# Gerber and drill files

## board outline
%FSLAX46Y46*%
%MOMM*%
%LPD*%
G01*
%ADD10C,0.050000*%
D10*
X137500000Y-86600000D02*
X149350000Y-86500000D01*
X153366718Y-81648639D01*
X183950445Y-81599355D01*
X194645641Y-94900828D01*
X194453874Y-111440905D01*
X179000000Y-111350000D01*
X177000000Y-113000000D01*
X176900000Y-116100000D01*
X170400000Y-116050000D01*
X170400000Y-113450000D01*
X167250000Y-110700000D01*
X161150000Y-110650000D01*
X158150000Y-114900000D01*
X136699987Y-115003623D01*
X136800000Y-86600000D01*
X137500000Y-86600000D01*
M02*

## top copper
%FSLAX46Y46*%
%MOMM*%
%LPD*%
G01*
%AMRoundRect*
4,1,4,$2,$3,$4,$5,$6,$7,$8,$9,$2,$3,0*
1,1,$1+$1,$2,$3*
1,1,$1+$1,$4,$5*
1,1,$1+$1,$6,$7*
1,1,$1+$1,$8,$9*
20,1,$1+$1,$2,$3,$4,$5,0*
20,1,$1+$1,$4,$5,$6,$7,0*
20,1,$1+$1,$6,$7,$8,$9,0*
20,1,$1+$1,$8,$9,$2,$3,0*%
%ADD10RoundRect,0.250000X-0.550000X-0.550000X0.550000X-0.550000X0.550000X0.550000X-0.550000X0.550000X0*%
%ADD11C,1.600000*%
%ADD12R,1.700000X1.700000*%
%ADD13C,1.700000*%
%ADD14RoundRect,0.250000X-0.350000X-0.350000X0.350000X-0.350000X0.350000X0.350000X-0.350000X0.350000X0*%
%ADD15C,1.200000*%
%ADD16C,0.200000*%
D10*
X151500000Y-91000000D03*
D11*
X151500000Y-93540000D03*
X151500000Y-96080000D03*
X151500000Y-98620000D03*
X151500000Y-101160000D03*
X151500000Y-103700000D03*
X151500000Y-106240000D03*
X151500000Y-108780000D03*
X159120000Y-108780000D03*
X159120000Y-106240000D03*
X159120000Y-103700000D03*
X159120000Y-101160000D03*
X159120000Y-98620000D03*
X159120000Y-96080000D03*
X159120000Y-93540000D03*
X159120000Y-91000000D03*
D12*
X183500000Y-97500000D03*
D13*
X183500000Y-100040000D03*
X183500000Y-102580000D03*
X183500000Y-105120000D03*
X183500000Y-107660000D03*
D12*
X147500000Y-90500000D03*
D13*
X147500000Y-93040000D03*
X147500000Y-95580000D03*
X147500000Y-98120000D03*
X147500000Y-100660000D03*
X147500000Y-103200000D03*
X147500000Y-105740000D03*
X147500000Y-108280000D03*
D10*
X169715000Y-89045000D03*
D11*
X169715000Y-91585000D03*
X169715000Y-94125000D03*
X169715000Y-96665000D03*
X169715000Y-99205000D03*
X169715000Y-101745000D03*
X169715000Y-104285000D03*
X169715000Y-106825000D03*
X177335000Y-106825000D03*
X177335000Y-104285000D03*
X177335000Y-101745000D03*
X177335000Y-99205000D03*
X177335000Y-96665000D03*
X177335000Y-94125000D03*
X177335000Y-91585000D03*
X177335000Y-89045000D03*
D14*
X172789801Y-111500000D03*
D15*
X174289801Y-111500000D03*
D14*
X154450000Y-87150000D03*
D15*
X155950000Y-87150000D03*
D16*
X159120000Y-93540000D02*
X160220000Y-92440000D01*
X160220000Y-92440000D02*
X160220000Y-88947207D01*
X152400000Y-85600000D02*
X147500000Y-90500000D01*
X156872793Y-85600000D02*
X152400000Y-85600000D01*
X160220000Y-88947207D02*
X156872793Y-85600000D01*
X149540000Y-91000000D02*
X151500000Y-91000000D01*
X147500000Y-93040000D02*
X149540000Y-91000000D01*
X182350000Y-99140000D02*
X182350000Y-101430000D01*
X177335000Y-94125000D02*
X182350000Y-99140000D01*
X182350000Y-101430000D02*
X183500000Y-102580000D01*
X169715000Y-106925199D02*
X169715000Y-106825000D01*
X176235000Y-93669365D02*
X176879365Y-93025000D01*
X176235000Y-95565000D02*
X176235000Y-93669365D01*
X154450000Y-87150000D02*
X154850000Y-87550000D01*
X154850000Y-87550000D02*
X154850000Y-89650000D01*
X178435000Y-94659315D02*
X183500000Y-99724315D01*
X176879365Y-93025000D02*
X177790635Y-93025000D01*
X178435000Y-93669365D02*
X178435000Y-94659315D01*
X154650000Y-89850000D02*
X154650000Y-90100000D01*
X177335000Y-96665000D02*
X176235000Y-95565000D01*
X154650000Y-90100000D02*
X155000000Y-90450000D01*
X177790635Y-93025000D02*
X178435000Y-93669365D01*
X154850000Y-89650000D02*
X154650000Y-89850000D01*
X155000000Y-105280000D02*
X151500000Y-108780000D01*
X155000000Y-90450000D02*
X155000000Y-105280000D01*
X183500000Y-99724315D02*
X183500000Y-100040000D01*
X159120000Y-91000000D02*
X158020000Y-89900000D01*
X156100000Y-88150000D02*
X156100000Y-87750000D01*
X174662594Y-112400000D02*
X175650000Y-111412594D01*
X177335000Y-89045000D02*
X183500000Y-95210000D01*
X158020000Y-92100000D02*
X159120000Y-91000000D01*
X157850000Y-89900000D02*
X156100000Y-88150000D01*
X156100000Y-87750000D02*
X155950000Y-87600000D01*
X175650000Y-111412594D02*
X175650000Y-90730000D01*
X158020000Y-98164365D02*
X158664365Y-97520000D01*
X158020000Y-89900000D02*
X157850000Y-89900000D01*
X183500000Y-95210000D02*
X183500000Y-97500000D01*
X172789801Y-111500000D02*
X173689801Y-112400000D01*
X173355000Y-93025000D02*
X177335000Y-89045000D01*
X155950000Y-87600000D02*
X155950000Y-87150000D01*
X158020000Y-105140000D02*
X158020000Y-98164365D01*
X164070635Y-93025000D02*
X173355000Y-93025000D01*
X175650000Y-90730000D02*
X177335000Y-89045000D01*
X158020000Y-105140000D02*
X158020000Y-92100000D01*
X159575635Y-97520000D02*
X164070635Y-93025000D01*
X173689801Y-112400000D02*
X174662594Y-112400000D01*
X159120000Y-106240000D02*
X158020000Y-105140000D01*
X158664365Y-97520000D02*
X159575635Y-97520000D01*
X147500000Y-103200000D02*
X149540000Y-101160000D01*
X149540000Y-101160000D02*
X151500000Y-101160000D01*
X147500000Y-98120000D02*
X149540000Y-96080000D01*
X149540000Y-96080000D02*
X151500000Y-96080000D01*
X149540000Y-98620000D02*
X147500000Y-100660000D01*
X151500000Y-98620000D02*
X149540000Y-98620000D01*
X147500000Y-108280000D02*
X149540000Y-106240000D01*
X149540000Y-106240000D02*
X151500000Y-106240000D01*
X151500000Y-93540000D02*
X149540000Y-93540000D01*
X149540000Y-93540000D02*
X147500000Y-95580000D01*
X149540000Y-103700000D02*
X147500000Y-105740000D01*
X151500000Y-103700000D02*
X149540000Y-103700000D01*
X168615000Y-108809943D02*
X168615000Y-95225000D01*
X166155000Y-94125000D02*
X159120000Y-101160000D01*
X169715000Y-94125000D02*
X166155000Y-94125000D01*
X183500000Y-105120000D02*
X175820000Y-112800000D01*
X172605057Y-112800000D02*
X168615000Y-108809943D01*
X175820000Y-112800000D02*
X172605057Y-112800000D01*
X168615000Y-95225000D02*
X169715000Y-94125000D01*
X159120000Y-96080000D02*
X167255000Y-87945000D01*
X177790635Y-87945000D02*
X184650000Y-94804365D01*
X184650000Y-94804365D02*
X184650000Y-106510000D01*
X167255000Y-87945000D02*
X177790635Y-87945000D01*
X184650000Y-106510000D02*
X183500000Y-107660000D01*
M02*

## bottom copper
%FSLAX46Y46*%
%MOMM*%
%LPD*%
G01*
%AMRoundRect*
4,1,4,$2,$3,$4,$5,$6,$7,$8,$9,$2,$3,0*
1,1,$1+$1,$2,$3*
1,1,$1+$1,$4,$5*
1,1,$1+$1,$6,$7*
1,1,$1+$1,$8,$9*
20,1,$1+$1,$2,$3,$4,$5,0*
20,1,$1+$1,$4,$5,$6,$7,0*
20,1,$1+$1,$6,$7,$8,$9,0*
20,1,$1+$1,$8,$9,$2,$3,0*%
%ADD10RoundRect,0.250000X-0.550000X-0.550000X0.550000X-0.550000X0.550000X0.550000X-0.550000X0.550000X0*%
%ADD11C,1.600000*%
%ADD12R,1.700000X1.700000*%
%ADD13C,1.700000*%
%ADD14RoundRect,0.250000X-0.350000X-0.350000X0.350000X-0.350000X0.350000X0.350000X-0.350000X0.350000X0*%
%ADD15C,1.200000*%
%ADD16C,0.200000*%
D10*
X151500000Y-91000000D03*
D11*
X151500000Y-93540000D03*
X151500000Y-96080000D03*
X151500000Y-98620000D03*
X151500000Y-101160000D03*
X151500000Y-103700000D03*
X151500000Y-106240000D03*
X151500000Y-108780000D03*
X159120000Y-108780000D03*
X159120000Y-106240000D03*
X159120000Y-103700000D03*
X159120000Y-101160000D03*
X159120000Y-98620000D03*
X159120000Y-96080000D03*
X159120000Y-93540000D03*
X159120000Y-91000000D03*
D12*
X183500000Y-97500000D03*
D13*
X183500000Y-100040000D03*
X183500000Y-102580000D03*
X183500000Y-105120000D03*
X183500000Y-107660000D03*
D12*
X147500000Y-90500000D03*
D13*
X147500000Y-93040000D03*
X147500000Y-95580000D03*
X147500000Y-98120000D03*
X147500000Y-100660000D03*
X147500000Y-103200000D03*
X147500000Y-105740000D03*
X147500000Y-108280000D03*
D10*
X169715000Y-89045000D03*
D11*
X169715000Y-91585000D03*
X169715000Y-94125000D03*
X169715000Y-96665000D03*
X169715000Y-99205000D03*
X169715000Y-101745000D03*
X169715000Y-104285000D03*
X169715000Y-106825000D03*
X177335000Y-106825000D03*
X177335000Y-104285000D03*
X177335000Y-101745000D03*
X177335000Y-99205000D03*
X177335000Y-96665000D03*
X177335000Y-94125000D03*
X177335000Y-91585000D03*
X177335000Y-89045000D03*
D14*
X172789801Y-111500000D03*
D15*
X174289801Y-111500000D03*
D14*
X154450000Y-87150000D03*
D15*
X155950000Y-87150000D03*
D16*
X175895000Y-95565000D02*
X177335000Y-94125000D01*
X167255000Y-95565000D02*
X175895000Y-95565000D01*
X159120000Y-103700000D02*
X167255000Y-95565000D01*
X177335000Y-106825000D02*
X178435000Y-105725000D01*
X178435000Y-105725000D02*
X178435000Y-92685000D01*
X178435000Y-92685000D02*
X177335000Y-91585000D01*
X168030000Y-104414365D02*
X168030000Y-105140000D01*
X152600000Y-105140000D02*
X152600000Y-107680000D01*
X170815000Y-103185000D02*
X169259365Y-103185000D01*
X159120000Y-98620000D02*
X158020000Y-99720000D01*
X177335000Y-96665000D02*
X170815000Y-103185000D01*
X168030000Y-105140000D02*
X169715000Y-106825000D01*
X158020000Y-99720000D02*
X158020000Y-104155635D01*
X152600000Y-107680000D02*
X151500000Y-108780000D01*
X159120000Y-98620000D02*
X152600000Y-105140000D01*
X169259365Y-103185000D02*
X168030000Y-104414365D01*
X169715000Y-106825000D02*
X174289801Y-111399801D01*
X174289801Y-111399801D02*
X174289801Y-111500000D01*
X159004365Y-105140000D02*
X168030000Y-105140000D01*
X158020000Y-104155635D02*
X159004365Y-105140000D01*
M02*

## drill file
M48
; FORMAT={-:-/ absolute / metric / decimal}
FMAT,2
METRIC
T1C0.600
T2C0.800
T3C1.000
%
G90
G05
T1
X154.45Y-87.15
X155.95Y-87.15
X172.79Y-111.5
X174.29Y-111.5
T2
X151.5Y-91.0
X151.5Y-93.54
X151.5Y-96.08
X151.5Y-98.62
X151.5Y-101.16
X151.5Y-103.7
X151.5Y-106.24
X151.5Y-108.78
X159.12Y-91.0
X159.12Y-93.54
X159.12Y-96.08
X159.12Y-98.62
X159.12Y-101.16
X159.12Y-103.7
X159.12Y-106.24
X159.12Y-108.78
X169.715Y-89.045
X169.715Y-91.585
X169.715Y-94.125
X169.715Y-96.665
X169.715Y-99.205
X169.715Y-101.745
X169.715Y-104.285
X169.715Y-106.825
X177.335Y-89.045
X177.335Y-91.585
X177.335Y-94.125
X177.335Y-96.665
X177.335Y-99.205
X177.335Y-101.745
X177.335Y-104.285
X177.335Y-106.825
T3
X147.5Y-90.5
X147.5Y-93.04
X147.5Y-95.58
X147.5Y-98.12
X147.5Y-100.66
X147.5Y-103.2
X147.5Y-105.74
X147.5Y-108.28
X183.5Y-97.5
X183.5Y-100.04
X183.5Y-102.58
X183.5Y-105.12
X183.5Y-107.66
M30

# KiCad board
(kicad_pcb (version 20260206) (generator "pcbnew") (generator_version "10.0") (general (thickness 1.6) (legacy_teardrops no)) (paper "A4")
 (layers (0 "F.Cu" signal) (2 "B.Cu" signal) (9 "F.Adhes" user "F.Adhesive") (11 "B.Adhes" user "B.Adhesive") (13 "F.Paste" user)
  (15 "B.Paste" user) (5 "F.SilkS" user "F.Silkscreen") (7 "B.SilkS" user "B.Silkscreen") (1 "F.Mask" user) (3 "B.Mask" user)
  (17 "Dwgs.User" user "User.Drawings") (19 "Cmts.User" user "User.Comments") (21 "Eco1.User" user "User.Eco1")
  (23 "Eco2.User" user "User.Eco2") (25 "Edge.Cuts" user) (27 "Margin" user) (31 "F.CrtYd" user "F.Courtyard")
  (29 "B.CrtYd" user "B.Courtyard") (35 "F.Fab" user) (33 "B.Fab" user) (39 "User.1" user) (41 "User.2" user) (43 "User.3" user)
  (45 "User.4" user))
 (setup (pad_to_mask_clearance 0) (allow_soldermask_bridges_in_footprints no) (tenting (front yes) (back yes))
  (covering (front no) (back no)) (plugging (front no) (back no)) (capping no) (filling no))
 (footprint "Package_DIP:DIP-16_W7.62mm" (layer "F.Cu") (at 151.5 91)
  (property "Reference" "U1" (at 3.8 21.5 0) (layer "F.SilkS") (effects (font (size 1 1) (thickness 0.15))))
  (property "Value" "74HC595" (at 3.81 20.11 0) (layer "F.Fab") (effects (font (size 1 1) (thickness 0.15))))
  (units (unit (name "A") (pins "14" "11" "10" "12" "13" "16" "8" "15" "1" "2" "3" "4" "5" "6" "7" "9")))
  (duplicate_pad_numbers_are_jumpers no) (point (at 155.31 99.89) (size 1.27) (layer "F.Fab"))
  (pad "1" thru_hole roundrect (at 0 0) (size 1.6 1.6) (drill 0.8) (layers "*.Cu" "*.Mask") (remove_unused_layers no)
   (roundrect_rratio 0.15625) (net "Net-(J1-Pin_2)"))
  (pad "2" thru_hole circle (at 0 2.54) (size 1.6 1.6) (drill 0.8) (layers "*.Cu" "*.Mask") (remove_unused_layers no) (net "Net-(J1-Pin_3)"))
  (pad "3" thru_hole circle (at 0 5.08) (size 1.6 1.6) (drill 0.8) (layers "*.Cu" "*.Mask") (remove_unused_layers no) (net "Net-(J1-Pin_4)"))
  (pad "4" thru_hole circle (at 0 7.62) (size 1.6 1.6) (drill 0.8) (layers "*.Cu" "*.Mask") (remove_unused_layers no) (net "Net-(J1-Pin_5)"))
  (pad "5" thru_hole circle (at 0 10.16) (size 1.6 1.6) (drill 0.8) (layers "*.Cu" "*.Mask") (remove_unused_layers no)
   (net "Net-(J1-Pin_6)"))
  (pad "6" thru_hole circle (at 0 12.7) (size 1.6 1.6) (drill 0.8) (layers "*.Cu" "*.Mask") (remove_unused_layers no) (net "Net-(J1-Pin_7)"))
  (pad "7" thru_hole circle (at 0 15.24) (size 1.6 1.6) (drill 0.8) (layers "*.Cu" "*.Mask") (remove_unused_layers no)
   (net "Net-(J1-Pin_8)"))
  (pad "8" thru_hole circle (at 0 17.78) (size 1.6 1.6) (drill 0.8) (layers "*.Cu" "*.Mask") (remove_unused_layers no) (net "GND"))
  (pad "9" thru_hole circle (at 7.62 17.78) (size 1.6 1.6) (drill 0.8) (layers "*.Cu" "*.Mask") (remove_unused_layers no)
   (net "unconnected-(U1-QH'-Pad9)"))
  (pad "10" thru_hole circle (at 7.62 15.24) (size 1.6 1.6) (drill 0.8) (layers "*.Cu" "*.Mask") (remove_unused_layers no) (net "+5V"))
  (pad "11" thru_hole circle (at 7.62 12.7) (size 1.6 1.6) (drill 0.8) (layers "*.Cu" "*.Mask") (remove_unused_layers no) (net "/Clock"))
  (pad "12" thru_hole circle (at 7.62 10.16) (size 1.6 1.6) (drill 0.8) (layers "*.Cu" "*.Mask") (remove_unused_layers no)
   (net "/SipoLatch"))
  (pad "13" thru_hole circle (at 7.62 7.62) (size 1.6 1.6) (drill 0.8) (layers "*.Cu" "*.Mask") (remove_unused_layers no) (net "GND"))
  (pad "14" thru_hole circle (at 7.62 5.08) (size 1.6 1.6) (drill 0.8) (layers "*.Cu" "*.Mask") (remove_unused_layers no) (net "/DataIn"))
  (pad "15" thru_hole circle (at 7.62 2.54) (size 1.6 1.6) (drill 0.8) (layers "*.Cu" "*.Mask") (remove_unused_layers no)
   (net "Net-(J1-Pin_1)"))
  (pad "16" thru_hole circle (at 7.62 0) (size 1.6 1.6) (drill 0.8) (layers "*.Cu" "*.Mask") (remove_unused_layers no) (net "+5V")))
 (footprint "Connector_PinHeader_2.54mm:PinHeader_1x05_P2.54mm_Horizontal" (layer "F.Cu") (at 183.5 97.5)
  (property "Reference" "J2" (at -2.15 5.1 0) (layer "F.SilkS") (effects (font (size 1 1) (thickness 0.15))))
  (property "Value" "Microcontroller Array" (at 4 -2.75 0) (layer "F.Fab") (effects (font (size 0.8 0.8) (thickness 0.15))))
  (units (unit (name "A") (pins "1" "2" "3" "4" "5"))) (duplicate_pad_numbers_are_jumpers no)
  (pad "1" thru_hole rect (at 0 0) (size 1.7 1.7) (drill 1) (layers "*.Cu" "*.Mask") (remove_unused_layers no) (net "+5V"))
  (pad "2" thru_hole circle (at 0 2.54) (size 1.7 1.7) (drill 1) (layers "*.Cu" "*.Mask") (remove_unused_layers no) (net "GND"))
  (pad "3" thru_hole circle (at 0 5.08) (size 1.7 1.7) (drill 1) (layers "*.Cu" "*.Mask") (remove_unused_layers no) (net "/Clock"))
  (pad "4" thru_hole circle (at 0 7.62) (size 1.7 1.7) (drill 1) (layers "*.Cu" "*.Mask") (remove_unused_layers no) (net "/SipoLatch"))
  (pad "5" thru_hole circle (at 0 10.16) (size 1.7 1.7) (drill 1) (layers "*.Cu" "*.Mask") (remove_unused_layers no) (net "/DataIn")))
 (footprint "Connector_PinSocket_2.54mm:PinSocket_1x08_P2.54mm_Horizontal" (layer "F.Cu") (at 147.5 90.5)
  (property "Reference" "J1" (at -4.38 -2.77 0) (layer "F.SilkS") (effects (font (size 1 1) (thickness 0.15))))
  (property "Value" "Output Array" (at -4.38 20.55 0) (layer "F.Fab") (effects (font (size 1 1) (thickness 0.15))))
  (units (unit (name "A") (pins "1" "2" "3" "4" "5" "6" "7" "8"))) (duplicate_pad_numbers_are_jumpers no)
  (pad "1" thru_hole rect (at 0 0) (size 1.7 1.7) (drill 1) (layers "*.Cu" "*.Mask") (remove_unused_layers no) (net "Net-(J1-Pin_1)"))
  (pad "2" thru_hole circle (at 0 2.54) (size 1.7 1.7) (drill 1) (layers "*.Cu" "*.Mask") (remove_unused_layers no) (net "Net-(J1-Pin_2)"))
  (pad "3" thru_hole circle (at 0 5.08) (size 1.7 1.7) (drill 1) (layers "*.Cu" "*.Mask") (remove_unused_layers no) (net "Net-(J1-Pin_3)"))
  (pad "4" thru_hole circle (at 0 7.62) (size 1.7 1.7) (drill 1) (layers "*.Cu" "*.Mask") (remove_unused_layers no) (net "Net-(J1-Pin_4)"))
  (pad "5" thru_hole circle (at 0 10.16) (size 1.7 1.7) (drill 1) (layers "*.Cu" "*.Mask") (remove_unused_layers no) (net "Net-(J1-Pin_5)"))
  (pad "6" thru_hole circle (at 0 12.7) (size 1.7 1.7) (drill 1) (layers "*.Cu" "*.Mask") (remove_unused_layers no) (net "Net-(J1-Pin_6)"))
  (pad "7" thru_hole circle (at 0 15.24) (size 1.7 1.7) (drill 1) (layers "*.Cu" "*.Mask") (remove_unused_layers no) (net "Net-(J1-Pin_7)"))
  (pad "8" thru_hole circle (at 0 17.78) (size 1.7 1.7) (drill 1) (layers "*.Cu" "*.Mask") (remove_unused_layers no) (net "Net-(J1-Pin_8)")))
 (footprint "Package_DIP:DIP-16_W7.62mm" (layer "F.Cu") (at 169.715 89.045)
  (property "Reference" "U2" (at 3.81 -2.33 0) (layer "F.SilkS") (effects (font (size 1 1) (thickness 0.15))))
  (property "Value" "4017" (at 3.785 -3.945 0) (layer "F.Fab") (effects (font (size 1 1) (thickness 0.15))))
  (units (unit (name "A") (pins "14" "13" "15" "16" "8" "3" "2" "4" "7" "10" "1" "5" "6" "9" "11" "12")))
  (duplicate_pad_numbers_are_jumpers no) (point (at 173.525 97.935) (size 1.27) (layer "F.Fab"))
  (pad "1" thru_hole roundrect (at 0 0) (size 1.6 1.6) (drill 0.8) (layers "*.Cu" "*.Mask") (remove_unused_layers no)
   (roundrect_rratio 0.15625) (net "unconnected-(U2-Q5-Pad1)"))
  (pad "2" thru_hole circle (at 0 2.54) (size 1.6 1.6) (drill 0.8) (layers "*.Cu" "*.Mask") (remove_unused_layers no)
   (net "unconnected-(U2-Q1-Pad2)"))
  (pad "3" thru_hole circle (at 0 5.08) (size 1.6 1.6) (drill 0.8) (layers "*.Cu" "*.Mask") (remove_unused_layers no) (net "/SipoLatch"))
  (pad "4" thru_hole circle (at 0 7.62) (size 1.6 1.6) (drill 0.8) (layers "*.Cu" "*.Mask") (remove_unused_layers no)
   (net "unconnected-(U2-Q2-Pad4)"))
  (pad "5" thru_hole circle (at 0 10.16) (size 1.6 1.6) (drill 0.8) (layers "*.Cu" "*.Mask") (remove_unused_layers no)
   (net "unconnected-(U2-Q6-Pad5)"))
  (pad "6" thru_hole circle (at 0 12.7) (size 1.6 1.6) (drill 0.8) (layers "*.Cu" "*.Mask") (remove_unused_layers no)
   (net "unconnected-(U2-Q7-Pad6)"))
  (pad "7" thru_hole circle (at 0 15.24) (size 1.6 1.6) (drill 0.8) (layers "*.Cu" "*.Mask") (remove_unused_layers no)
   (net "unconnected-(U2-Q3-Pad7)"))
  (pad "8" thru_hole circle (at 0 17.78) (size 1.6 1.6) (drill 0.8) (layers "*.Cu" "*.Mask") (remove_unused_layers no) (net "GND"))
  (pad "9" thru_hole circle (at 7.62 17.78) (size 1.6 1.6) (drill 0.8) (layers "*.Cu" "*.Mask") (remove_unused_layers no)
   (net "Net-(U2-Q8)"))
  (pad "10" thru_hole circle (at 7.62 15.24) (size 1.6 1.6) (drill 0.8) (layers "*.Cu" "*.Mask") (remove_unused_layers no)
   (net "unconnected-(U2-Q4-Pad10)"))
  (pad "11" thru_hole circle (at 7.62 12.7) (size 1.6 1.6) (drill 0.8) (layers "*.Cu" "*.Mask") (remove_unused_layers no)
   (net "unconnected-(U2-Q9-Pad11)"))
  (pad "12" thru_hole circle (at 7.62 10.16) (size 1.6 1.6) (drill 0.8) (layers "*.Cu" "*.Mask") (remove_unused_layers no)
   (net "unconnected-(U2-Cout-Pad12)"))
  (pad "13" thru_hole circle (at 7.62 7.62) (size 1.6 1.6) (drill 0.8) (layers "*.Cu" "*.Mask") (remove_unused_layers no) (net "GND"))
  (pad "14" thru_hole circle (at 7.62 5.08) (size 1.6 1.6) (drill 0.8) (layers "*.Cu" "*.Mask") (remove_unused_layers no) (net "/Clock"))
  (pad "15" thru_hole circle (at 7.62 2.54) (size 1.6 1.6) (drill 0.8) (layers "*.Cu" "*.Mask") (remove_unused_layers no)
   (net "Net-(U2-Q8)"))
  (pad "16" thru_hole circle (at 7.62 0) (size 1.6 1.6) (drill 0.8) (layers "*.Cu" "*.Mask") (remove_unused_layers no) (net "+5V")))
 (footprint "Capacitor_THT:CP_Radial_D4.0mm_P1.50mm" (layer "F.Cu") (at 172.789801 111.5)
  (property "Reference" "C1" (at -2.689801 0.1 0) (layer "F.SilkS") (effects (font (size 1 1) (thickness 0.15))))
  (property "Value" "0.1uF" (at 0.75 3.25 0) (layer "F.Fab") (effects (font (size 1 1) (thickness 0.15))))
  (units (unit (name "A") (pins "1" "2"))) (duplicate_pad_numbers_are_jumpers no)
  (pad "1" thru_hole roundrect (at 0 0) (size 1.2 1.2) (drill 0.6) (layers "*.Cu" "*.Mask") (remove_unused_layers no)
   (roundrect_rratio 0.208333) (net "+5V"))
  (pad "2" thru_hole circle (at 1.5 0) (size 1.2 1.2) (drill 0.6) (layers "*.Cu" "*.Mask") (remove_unused_layers no) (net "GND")))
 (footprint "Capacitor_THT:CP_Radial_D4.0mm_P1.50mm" (layer "F.Cu") (at 154.45 87.15)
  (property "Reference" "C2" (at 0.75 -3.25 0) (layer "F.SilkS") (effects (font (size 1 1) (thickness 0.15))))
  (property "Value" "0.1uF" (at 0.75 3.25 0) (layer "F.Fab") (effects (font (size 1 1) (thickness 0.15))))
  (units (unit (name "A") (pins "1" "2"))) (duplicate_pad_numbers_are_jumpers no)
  (pad "1" thru_hole roundrect (at 0 0) (size 1.2 1.2) (drill 0.6) (layers "*.Cu" "*.Mask") (remove_unused_layers no)
   (roundrect_rratio 0.208333) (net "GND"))
  (pad "2" thru_hole circle (at 1.5 0) (size 1.2 1.2) (drill 0.6) (layers "*.Cu" "*.Mask") (remove_unused_layers no) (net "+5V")))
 (gr_poly
  (pts (xy 137.5 86.6) (xy 149.35 86.5) (xy 153.366718 81.648639) (xy 183.950445 81.599355) (xy 194.645641 94.900828)
   (xy 194.453874 111.440905) (xy 179 111.35) (xy 177 113) (xy 176.9 116.1) (xy 170.4 116.05) (xy 170.4 113.45) (xy 167.25 110.7)
   (xy 161.15 110.65) (xy 158.15 114.9) (xy 136.699987 115.003623) (xy 136.8 86.6))
  (stroke (width 0.05) (type solid)) (fill no) (layer "Edge.Cuts"))
 (segment (start 159.12 93.54) (end 160.22 92.44) (width 0.2) (layer "F.Cu") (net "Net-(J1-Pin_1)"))
 (segment (start 160.22 92.44) (end 160.22 88.947207) (width 0.2) (layer "F.Cu") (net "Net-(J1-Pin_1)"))
 (segment (start 152.4 85.6) (end 147.5 90.5) (width 0.2) (layer "F.Cu") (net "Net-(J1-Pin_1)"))
 (segment (start 156.872793 85.6) (end 152.4 85.6) (width 0.2) (layer "F.Cu") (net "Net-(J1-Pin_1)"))
 (segment (start 160.22 88.947207) (end 156.872793 85.6) (width 0.2) (layer "F.Cu") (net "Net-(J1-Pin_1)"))
 (segment (start 149.54 91) (end 151.5 91) (width 0.2) (layer "F.Cu") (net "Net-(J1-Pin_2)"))
 (segment (start 147.5 93.04) (end 149.54 91) (width 0.2) (layer "F.Cu") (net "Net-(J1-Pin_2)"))
 (segment (start 182.35 99.14) (end 182.35 101.43) (width 0.2) (layer "F.Cu") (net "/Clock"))
 (segment (start 177.335 94.125) (end 182.35 99.14) (width 0.2) (layer "F.Cu") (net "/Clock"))
 (segment (start 182.35 101.43) (end 183.5 102.58) (width 0.2) (layer "F.Cu") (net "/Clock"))
 (segment (start 175.895 95.565) (end 177.335 94.125) (width 0.2) (layer "B.Cu") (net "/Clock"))
 (segment (start 167.255 95.565) (end 175.895 95.565) (width 0.2) (layer "B.Cu") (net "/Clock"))
 (segment (start 159.12 103.7) (end 167.255 95.565) (width 0.2) (layer "B.Cu") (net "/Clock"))
 (segment (start 177.335 106.825) (end 178.435 105.725) (width 0.2) (layer "B.Cu") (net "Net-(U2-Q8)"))
 (segment (start 178.435 105.725) (end 178.435 92.685) (width 0.2) (layer "B.Cu") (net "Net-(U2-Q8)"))
 (segment (start 178.435 92.685) (end 177.335 91.585) (width 0.2) (layer "B.Cu") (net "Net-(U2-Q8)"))
 (segment (start 169.715 106.925199) (end 169.715 106.825) (width 0.2) (layer "F.Cu") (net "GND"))
 (segment (start 176.235 93.669365) (end 176.879365 93.025) (width 0.2) (layer "F.Cu") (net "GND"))
 (segment (start 176.235 95.565) (end 176.235 93.669365) (width 0.2) (layer "F.Cu") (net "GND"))
 (segment (start 154.45 87.15) (end 154.85 87.55) (width 0.2) (layer "F.Cu") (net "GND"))
 (segment (start 154.85 87.55) (end 154.85 89.65) (width 0.2) (layer "F.Cu") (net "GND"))
 (segment (start 178.435 94.659315) (end 183.5 99.724315) (width 0.2) (layer "F.Cu") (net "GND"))
 (segment (start 176.879365 93.025) (end 177.790635 93.025) (width 0.2) (layer "F.Cu") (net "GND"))
 (segment (start 178.435 93.669365) (end 178.435 94.659315) (width 0.2) (layer "F.Cu") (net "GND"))
 (segment (start 154.65 89.85) (end 154.65 90.1) (width 0.2) (layer "F.Cu") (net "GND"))
 (segment (start 177.335 96.665) (end 176.235 95.565) (width 0.2) (layer "F.Cu") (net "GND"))
 (segment (start 154.65 90.1) (end 155 90.45) (width 0.2) (layer "F.Cu") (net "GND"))
 (segment (start 177.790635 93.025) (end 178.435 93.669365) (width 0.2) (layer "F.Cu") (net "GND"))
 (segment (start 154.85 89.65) (end 154.65 89.85) (width 0.2) (layer "F.Cu") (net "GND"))
 (segment (start 155 105.28) (end 151.5 108.78) (width 0.2) (layer "F.Cu") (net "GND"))
 (segment (start 155 90.45) (end 155 105.28) (width 0.2) (layer "F.Cu") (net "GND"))
 (segment (start 183.5 99.724315) (end 183.5 100.04) (width 0.2) (layer "F.Cu") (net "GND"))
 (segment (start 168.03 104.414365) (end 168.03 105.14) (width 0.2) (layer "B.Cu") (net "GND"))
 (segment (start 152.6 105.14) (end 152.6 107.68) (width 0.2) (layer "B.Cu") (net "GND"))
 (segment (start 170.815 103.185) (end 169.259365 103.185) (width 0.2) (layer "B.Cu") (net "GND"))
 (segment (start 159.12 98.62) (end 158.02 99.72) (width 0.2) (layer "B.Cu") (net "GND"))
 (segment (start 177.335 96.665) (end 170.815 103.185) (width 0.2) (layer "B.Cu") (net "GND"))
 (segment (start 168.03 105.14) (end 169.715 106.825) (width 0.2) (layer "B.Cu") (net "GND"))
 (segment (start 158.02 99.72) (end 158.02 104.155635) (width 0.2) (layer "B.Cu") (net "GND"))
 (segment (start 152.6 107.68) (end 151.5 108.78) (width 0.2) (layer "B.Cu") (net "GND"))
 (segment (start 159.12 98.62) (end 152.6 105.14) (width 0.2) (layer "B.Cu") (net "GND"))
 (segment (start 169.259365 103.185) (end 168.03 104.414365) (width 0.2) (layer "B.Cu") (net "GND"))
 (segment (start 169.715 106.825) (end 174.289801 111.399801) (width 0.2) (layer "B.Cu") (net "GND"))
 (segment (start 174.289801 111.399801) (end 174.289801 111.5) (width 0.2) (layer "B.Cu") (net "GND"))
 (segment (start 159.004365 105.14) (end 168.03 105.14) (width 0.2) (layer "B.Cu") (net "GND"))
 (segment (start 158.02 104.155635) (end 159.004365 105.14) (width 0.2) (layer "B.Cu") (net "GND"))
 (segment (start 159.12 91) (end 158.02 89.9) (width 0.2) (layer "F.Cu") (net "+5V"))
 (segment (start 156.1 88.15) (end 156.1 87.75) (width 0.2) (layer "F.Cu") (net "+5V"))
 (segment (start 174.662594 112.4) (end 175.65 111.412594) (width 0.2) (layer "F.Cu") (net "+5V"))
 (segment (start 177.335 89.045) (end 183.5 95.21) (width 0.2) (layer "F.Cu") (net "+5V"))
 (segment (start 158.02 92.1) (end 159.12 91) (width 0.2) (layer "F.Cu") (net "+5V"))
 (segment (start 157.85 89.9) (end 156.1 88.15) (width 0.2) (layer "F.Cu") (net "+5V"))
 (segment (start 156.1 87.75) (end 155.95 87.6) (width 0.2) (layer "F.Cu") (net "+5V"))
 (segment (start 175.65 111.412594) (end 175.65 90.73) (width 0.2) (layer "F.Cu") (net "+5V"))
 (segment (start 158.02 98.164365) (end 158.664365 97.52) (width 0.2) (layer "F.Cu") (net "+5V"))
 (segment (start 158.02 89.9) (end 157.85 89.9) (width 0.2) (layer "F.Cu") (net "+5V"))
 (segment (start 183.5 95.21) (end 183.5 97.5) (width 0.2) (layer "F.Cu") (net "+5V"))
 (segment (start 172.789801 111.5) (end 173.689801 112.4) (width 0.2) (layer "F.Cu") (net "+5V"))
 (segment (start 173.355 93.025) (end 177.335 89.045) (width 0.2) (layer "F.Cu") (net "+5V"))
 (segment (start 155.95 87.6) (end 155.95 87.15) (width 0.2) (layer "F.Cu") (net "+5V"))
 (segment (start 158.02 105.14) (end 158.02 98.164365) (width 0.2) (layer "F.Cu") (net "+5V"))
 (segment (start 164.070635 93.025) (end 173.355 93.025) (width 0.2) (layer "F.Cu") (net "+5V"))
 (segment (start 175.65 90.73) (end 177.335 89.045) (width 0.2) (layer "F.Cu") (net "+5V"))
 (segment (start 158.02 105.14) (end 158.02 92.1) (width 0.2) (layer "F.Cu") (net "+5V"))
 (segment (start 159.575635 97.52) (end 164.070635 93.025) (width 0.2) (layer "F.Cu") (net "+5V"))
 (segment (start 173.689801 112.4) (end 174.662594 112.4) (width 0.2) (layer "F.Cu") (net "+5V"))
 (segment (start 159.12 106.24) (end 158.02 105.14) (width 0.2) (layer "F.Cu") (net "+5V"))
 (segment (start 158.664365 97.52) (end 159.575635 97.52) (width 0.2) (layer "F.Cu") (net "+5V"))
 (segment (start 147.5 103.2) (end 149.54 101.16) (width 0.2) (layer "F.Cu") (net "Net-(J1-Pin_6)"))
 (segment (start 149.54 101.16) (end 151.5 101.16) (width 0.2) (layer "F.Cu") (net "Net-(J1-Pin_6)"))
 (segment (start 147.5 98.12) (end 149.54 96.08) (width 0.2) (layer "F.Cu") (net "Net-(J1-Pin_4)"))
 (segment (start 149.54 96.08) (end 151.5 96.08) (width 0.2) (layer "F.Cu") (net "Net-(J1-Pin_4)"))
 (segment (start 149.54 98.62) (end 147.5 100.66) (width 0.2) (layer "F.Cu") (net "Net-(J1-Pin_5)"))
 (segment (start 151.5 98.62) (end 149.54 98.62) (width 0.2) (layer "F.Cu") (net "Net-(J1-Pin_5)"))
 (segment (start 147.5 108.28) (end 149.54 106.24) (width 0.2) (layer "F.Cu") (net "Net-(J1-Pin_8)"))
 (segment (start 149.54 106.24) (end 151.5 106.24) (width 0.2) (layer "F.Cu") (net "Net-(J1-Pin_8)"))
 (segment (start 151.5 93.54) (end 149.54 93.54) (width 0.2) (layer "F.Cu") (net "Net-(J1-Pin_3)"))
 (segment (start 149.54 93.54) (end 147.5 95.58) (width 0.2) (layer "F.Cu") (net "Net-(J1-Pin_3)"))
 (segment (start 149.54 103.7) (end 147.5 105.74) (width 0.2) (layer "F.Cu") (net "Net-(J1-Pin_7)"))
 (segment (start 151.5 103.7) (end 149.54 103.7) (width 0.2) (layer "F.Cu") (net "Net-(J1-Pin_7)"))
 (segment (start 168.615 108.809943) (end 168.615 95.225) (width 0.2) (layer "F.Cu") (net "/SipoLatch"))
 (segment (start 166.155 94.125) (end 159.12 101.16) (width 0.2) (layer "F.Cu") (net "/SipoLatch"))
 (segment (start 169.715 94.125) (end 166.155 94.125) (width 0.2) (layer "F.Cu") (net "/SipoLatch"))
 (segment (start 183.5 105.12) (end 175.82 112.8) (width 0.2) (layer "F.Cu") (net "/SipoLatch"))
 (segment (start 172.605057 112.8) (end 168.615 108.809943) (width 0.2) (layer "F.Cu") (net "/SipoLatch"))
 (segment (start 175.82 112.8) (end 172.605057 112.8) (width 0.2) (layer "F.Cu") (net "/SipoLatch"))
 (segment (start 168.615 95.225) (end 169.715 94.125) (width 0.2) (layer "F.Cu") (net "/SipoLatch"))
 (segment (start 159.12 96.08) (end 167.255 87.945) (width 0.2) (layer "F.Cu") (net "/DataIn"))
 (segment (start 177.790635 87.945) (end 184.65 94.804365) (width 0.2) (layer "F.Cu") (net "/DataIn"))
 (segment (start 184.65 94.804365) (end 184.65 106.51) (width 0.2) (layer "F.Cu") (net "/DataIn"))
 (segment (start 167.255 87.945) (end 177.790635 87.945) (width 0.2) (layer "F.Cu") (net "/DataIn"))
 (segment (start 184.65 106.51) (end 183.5 107.66) (width 0.2) (layer "F.Cu") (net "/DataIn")))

